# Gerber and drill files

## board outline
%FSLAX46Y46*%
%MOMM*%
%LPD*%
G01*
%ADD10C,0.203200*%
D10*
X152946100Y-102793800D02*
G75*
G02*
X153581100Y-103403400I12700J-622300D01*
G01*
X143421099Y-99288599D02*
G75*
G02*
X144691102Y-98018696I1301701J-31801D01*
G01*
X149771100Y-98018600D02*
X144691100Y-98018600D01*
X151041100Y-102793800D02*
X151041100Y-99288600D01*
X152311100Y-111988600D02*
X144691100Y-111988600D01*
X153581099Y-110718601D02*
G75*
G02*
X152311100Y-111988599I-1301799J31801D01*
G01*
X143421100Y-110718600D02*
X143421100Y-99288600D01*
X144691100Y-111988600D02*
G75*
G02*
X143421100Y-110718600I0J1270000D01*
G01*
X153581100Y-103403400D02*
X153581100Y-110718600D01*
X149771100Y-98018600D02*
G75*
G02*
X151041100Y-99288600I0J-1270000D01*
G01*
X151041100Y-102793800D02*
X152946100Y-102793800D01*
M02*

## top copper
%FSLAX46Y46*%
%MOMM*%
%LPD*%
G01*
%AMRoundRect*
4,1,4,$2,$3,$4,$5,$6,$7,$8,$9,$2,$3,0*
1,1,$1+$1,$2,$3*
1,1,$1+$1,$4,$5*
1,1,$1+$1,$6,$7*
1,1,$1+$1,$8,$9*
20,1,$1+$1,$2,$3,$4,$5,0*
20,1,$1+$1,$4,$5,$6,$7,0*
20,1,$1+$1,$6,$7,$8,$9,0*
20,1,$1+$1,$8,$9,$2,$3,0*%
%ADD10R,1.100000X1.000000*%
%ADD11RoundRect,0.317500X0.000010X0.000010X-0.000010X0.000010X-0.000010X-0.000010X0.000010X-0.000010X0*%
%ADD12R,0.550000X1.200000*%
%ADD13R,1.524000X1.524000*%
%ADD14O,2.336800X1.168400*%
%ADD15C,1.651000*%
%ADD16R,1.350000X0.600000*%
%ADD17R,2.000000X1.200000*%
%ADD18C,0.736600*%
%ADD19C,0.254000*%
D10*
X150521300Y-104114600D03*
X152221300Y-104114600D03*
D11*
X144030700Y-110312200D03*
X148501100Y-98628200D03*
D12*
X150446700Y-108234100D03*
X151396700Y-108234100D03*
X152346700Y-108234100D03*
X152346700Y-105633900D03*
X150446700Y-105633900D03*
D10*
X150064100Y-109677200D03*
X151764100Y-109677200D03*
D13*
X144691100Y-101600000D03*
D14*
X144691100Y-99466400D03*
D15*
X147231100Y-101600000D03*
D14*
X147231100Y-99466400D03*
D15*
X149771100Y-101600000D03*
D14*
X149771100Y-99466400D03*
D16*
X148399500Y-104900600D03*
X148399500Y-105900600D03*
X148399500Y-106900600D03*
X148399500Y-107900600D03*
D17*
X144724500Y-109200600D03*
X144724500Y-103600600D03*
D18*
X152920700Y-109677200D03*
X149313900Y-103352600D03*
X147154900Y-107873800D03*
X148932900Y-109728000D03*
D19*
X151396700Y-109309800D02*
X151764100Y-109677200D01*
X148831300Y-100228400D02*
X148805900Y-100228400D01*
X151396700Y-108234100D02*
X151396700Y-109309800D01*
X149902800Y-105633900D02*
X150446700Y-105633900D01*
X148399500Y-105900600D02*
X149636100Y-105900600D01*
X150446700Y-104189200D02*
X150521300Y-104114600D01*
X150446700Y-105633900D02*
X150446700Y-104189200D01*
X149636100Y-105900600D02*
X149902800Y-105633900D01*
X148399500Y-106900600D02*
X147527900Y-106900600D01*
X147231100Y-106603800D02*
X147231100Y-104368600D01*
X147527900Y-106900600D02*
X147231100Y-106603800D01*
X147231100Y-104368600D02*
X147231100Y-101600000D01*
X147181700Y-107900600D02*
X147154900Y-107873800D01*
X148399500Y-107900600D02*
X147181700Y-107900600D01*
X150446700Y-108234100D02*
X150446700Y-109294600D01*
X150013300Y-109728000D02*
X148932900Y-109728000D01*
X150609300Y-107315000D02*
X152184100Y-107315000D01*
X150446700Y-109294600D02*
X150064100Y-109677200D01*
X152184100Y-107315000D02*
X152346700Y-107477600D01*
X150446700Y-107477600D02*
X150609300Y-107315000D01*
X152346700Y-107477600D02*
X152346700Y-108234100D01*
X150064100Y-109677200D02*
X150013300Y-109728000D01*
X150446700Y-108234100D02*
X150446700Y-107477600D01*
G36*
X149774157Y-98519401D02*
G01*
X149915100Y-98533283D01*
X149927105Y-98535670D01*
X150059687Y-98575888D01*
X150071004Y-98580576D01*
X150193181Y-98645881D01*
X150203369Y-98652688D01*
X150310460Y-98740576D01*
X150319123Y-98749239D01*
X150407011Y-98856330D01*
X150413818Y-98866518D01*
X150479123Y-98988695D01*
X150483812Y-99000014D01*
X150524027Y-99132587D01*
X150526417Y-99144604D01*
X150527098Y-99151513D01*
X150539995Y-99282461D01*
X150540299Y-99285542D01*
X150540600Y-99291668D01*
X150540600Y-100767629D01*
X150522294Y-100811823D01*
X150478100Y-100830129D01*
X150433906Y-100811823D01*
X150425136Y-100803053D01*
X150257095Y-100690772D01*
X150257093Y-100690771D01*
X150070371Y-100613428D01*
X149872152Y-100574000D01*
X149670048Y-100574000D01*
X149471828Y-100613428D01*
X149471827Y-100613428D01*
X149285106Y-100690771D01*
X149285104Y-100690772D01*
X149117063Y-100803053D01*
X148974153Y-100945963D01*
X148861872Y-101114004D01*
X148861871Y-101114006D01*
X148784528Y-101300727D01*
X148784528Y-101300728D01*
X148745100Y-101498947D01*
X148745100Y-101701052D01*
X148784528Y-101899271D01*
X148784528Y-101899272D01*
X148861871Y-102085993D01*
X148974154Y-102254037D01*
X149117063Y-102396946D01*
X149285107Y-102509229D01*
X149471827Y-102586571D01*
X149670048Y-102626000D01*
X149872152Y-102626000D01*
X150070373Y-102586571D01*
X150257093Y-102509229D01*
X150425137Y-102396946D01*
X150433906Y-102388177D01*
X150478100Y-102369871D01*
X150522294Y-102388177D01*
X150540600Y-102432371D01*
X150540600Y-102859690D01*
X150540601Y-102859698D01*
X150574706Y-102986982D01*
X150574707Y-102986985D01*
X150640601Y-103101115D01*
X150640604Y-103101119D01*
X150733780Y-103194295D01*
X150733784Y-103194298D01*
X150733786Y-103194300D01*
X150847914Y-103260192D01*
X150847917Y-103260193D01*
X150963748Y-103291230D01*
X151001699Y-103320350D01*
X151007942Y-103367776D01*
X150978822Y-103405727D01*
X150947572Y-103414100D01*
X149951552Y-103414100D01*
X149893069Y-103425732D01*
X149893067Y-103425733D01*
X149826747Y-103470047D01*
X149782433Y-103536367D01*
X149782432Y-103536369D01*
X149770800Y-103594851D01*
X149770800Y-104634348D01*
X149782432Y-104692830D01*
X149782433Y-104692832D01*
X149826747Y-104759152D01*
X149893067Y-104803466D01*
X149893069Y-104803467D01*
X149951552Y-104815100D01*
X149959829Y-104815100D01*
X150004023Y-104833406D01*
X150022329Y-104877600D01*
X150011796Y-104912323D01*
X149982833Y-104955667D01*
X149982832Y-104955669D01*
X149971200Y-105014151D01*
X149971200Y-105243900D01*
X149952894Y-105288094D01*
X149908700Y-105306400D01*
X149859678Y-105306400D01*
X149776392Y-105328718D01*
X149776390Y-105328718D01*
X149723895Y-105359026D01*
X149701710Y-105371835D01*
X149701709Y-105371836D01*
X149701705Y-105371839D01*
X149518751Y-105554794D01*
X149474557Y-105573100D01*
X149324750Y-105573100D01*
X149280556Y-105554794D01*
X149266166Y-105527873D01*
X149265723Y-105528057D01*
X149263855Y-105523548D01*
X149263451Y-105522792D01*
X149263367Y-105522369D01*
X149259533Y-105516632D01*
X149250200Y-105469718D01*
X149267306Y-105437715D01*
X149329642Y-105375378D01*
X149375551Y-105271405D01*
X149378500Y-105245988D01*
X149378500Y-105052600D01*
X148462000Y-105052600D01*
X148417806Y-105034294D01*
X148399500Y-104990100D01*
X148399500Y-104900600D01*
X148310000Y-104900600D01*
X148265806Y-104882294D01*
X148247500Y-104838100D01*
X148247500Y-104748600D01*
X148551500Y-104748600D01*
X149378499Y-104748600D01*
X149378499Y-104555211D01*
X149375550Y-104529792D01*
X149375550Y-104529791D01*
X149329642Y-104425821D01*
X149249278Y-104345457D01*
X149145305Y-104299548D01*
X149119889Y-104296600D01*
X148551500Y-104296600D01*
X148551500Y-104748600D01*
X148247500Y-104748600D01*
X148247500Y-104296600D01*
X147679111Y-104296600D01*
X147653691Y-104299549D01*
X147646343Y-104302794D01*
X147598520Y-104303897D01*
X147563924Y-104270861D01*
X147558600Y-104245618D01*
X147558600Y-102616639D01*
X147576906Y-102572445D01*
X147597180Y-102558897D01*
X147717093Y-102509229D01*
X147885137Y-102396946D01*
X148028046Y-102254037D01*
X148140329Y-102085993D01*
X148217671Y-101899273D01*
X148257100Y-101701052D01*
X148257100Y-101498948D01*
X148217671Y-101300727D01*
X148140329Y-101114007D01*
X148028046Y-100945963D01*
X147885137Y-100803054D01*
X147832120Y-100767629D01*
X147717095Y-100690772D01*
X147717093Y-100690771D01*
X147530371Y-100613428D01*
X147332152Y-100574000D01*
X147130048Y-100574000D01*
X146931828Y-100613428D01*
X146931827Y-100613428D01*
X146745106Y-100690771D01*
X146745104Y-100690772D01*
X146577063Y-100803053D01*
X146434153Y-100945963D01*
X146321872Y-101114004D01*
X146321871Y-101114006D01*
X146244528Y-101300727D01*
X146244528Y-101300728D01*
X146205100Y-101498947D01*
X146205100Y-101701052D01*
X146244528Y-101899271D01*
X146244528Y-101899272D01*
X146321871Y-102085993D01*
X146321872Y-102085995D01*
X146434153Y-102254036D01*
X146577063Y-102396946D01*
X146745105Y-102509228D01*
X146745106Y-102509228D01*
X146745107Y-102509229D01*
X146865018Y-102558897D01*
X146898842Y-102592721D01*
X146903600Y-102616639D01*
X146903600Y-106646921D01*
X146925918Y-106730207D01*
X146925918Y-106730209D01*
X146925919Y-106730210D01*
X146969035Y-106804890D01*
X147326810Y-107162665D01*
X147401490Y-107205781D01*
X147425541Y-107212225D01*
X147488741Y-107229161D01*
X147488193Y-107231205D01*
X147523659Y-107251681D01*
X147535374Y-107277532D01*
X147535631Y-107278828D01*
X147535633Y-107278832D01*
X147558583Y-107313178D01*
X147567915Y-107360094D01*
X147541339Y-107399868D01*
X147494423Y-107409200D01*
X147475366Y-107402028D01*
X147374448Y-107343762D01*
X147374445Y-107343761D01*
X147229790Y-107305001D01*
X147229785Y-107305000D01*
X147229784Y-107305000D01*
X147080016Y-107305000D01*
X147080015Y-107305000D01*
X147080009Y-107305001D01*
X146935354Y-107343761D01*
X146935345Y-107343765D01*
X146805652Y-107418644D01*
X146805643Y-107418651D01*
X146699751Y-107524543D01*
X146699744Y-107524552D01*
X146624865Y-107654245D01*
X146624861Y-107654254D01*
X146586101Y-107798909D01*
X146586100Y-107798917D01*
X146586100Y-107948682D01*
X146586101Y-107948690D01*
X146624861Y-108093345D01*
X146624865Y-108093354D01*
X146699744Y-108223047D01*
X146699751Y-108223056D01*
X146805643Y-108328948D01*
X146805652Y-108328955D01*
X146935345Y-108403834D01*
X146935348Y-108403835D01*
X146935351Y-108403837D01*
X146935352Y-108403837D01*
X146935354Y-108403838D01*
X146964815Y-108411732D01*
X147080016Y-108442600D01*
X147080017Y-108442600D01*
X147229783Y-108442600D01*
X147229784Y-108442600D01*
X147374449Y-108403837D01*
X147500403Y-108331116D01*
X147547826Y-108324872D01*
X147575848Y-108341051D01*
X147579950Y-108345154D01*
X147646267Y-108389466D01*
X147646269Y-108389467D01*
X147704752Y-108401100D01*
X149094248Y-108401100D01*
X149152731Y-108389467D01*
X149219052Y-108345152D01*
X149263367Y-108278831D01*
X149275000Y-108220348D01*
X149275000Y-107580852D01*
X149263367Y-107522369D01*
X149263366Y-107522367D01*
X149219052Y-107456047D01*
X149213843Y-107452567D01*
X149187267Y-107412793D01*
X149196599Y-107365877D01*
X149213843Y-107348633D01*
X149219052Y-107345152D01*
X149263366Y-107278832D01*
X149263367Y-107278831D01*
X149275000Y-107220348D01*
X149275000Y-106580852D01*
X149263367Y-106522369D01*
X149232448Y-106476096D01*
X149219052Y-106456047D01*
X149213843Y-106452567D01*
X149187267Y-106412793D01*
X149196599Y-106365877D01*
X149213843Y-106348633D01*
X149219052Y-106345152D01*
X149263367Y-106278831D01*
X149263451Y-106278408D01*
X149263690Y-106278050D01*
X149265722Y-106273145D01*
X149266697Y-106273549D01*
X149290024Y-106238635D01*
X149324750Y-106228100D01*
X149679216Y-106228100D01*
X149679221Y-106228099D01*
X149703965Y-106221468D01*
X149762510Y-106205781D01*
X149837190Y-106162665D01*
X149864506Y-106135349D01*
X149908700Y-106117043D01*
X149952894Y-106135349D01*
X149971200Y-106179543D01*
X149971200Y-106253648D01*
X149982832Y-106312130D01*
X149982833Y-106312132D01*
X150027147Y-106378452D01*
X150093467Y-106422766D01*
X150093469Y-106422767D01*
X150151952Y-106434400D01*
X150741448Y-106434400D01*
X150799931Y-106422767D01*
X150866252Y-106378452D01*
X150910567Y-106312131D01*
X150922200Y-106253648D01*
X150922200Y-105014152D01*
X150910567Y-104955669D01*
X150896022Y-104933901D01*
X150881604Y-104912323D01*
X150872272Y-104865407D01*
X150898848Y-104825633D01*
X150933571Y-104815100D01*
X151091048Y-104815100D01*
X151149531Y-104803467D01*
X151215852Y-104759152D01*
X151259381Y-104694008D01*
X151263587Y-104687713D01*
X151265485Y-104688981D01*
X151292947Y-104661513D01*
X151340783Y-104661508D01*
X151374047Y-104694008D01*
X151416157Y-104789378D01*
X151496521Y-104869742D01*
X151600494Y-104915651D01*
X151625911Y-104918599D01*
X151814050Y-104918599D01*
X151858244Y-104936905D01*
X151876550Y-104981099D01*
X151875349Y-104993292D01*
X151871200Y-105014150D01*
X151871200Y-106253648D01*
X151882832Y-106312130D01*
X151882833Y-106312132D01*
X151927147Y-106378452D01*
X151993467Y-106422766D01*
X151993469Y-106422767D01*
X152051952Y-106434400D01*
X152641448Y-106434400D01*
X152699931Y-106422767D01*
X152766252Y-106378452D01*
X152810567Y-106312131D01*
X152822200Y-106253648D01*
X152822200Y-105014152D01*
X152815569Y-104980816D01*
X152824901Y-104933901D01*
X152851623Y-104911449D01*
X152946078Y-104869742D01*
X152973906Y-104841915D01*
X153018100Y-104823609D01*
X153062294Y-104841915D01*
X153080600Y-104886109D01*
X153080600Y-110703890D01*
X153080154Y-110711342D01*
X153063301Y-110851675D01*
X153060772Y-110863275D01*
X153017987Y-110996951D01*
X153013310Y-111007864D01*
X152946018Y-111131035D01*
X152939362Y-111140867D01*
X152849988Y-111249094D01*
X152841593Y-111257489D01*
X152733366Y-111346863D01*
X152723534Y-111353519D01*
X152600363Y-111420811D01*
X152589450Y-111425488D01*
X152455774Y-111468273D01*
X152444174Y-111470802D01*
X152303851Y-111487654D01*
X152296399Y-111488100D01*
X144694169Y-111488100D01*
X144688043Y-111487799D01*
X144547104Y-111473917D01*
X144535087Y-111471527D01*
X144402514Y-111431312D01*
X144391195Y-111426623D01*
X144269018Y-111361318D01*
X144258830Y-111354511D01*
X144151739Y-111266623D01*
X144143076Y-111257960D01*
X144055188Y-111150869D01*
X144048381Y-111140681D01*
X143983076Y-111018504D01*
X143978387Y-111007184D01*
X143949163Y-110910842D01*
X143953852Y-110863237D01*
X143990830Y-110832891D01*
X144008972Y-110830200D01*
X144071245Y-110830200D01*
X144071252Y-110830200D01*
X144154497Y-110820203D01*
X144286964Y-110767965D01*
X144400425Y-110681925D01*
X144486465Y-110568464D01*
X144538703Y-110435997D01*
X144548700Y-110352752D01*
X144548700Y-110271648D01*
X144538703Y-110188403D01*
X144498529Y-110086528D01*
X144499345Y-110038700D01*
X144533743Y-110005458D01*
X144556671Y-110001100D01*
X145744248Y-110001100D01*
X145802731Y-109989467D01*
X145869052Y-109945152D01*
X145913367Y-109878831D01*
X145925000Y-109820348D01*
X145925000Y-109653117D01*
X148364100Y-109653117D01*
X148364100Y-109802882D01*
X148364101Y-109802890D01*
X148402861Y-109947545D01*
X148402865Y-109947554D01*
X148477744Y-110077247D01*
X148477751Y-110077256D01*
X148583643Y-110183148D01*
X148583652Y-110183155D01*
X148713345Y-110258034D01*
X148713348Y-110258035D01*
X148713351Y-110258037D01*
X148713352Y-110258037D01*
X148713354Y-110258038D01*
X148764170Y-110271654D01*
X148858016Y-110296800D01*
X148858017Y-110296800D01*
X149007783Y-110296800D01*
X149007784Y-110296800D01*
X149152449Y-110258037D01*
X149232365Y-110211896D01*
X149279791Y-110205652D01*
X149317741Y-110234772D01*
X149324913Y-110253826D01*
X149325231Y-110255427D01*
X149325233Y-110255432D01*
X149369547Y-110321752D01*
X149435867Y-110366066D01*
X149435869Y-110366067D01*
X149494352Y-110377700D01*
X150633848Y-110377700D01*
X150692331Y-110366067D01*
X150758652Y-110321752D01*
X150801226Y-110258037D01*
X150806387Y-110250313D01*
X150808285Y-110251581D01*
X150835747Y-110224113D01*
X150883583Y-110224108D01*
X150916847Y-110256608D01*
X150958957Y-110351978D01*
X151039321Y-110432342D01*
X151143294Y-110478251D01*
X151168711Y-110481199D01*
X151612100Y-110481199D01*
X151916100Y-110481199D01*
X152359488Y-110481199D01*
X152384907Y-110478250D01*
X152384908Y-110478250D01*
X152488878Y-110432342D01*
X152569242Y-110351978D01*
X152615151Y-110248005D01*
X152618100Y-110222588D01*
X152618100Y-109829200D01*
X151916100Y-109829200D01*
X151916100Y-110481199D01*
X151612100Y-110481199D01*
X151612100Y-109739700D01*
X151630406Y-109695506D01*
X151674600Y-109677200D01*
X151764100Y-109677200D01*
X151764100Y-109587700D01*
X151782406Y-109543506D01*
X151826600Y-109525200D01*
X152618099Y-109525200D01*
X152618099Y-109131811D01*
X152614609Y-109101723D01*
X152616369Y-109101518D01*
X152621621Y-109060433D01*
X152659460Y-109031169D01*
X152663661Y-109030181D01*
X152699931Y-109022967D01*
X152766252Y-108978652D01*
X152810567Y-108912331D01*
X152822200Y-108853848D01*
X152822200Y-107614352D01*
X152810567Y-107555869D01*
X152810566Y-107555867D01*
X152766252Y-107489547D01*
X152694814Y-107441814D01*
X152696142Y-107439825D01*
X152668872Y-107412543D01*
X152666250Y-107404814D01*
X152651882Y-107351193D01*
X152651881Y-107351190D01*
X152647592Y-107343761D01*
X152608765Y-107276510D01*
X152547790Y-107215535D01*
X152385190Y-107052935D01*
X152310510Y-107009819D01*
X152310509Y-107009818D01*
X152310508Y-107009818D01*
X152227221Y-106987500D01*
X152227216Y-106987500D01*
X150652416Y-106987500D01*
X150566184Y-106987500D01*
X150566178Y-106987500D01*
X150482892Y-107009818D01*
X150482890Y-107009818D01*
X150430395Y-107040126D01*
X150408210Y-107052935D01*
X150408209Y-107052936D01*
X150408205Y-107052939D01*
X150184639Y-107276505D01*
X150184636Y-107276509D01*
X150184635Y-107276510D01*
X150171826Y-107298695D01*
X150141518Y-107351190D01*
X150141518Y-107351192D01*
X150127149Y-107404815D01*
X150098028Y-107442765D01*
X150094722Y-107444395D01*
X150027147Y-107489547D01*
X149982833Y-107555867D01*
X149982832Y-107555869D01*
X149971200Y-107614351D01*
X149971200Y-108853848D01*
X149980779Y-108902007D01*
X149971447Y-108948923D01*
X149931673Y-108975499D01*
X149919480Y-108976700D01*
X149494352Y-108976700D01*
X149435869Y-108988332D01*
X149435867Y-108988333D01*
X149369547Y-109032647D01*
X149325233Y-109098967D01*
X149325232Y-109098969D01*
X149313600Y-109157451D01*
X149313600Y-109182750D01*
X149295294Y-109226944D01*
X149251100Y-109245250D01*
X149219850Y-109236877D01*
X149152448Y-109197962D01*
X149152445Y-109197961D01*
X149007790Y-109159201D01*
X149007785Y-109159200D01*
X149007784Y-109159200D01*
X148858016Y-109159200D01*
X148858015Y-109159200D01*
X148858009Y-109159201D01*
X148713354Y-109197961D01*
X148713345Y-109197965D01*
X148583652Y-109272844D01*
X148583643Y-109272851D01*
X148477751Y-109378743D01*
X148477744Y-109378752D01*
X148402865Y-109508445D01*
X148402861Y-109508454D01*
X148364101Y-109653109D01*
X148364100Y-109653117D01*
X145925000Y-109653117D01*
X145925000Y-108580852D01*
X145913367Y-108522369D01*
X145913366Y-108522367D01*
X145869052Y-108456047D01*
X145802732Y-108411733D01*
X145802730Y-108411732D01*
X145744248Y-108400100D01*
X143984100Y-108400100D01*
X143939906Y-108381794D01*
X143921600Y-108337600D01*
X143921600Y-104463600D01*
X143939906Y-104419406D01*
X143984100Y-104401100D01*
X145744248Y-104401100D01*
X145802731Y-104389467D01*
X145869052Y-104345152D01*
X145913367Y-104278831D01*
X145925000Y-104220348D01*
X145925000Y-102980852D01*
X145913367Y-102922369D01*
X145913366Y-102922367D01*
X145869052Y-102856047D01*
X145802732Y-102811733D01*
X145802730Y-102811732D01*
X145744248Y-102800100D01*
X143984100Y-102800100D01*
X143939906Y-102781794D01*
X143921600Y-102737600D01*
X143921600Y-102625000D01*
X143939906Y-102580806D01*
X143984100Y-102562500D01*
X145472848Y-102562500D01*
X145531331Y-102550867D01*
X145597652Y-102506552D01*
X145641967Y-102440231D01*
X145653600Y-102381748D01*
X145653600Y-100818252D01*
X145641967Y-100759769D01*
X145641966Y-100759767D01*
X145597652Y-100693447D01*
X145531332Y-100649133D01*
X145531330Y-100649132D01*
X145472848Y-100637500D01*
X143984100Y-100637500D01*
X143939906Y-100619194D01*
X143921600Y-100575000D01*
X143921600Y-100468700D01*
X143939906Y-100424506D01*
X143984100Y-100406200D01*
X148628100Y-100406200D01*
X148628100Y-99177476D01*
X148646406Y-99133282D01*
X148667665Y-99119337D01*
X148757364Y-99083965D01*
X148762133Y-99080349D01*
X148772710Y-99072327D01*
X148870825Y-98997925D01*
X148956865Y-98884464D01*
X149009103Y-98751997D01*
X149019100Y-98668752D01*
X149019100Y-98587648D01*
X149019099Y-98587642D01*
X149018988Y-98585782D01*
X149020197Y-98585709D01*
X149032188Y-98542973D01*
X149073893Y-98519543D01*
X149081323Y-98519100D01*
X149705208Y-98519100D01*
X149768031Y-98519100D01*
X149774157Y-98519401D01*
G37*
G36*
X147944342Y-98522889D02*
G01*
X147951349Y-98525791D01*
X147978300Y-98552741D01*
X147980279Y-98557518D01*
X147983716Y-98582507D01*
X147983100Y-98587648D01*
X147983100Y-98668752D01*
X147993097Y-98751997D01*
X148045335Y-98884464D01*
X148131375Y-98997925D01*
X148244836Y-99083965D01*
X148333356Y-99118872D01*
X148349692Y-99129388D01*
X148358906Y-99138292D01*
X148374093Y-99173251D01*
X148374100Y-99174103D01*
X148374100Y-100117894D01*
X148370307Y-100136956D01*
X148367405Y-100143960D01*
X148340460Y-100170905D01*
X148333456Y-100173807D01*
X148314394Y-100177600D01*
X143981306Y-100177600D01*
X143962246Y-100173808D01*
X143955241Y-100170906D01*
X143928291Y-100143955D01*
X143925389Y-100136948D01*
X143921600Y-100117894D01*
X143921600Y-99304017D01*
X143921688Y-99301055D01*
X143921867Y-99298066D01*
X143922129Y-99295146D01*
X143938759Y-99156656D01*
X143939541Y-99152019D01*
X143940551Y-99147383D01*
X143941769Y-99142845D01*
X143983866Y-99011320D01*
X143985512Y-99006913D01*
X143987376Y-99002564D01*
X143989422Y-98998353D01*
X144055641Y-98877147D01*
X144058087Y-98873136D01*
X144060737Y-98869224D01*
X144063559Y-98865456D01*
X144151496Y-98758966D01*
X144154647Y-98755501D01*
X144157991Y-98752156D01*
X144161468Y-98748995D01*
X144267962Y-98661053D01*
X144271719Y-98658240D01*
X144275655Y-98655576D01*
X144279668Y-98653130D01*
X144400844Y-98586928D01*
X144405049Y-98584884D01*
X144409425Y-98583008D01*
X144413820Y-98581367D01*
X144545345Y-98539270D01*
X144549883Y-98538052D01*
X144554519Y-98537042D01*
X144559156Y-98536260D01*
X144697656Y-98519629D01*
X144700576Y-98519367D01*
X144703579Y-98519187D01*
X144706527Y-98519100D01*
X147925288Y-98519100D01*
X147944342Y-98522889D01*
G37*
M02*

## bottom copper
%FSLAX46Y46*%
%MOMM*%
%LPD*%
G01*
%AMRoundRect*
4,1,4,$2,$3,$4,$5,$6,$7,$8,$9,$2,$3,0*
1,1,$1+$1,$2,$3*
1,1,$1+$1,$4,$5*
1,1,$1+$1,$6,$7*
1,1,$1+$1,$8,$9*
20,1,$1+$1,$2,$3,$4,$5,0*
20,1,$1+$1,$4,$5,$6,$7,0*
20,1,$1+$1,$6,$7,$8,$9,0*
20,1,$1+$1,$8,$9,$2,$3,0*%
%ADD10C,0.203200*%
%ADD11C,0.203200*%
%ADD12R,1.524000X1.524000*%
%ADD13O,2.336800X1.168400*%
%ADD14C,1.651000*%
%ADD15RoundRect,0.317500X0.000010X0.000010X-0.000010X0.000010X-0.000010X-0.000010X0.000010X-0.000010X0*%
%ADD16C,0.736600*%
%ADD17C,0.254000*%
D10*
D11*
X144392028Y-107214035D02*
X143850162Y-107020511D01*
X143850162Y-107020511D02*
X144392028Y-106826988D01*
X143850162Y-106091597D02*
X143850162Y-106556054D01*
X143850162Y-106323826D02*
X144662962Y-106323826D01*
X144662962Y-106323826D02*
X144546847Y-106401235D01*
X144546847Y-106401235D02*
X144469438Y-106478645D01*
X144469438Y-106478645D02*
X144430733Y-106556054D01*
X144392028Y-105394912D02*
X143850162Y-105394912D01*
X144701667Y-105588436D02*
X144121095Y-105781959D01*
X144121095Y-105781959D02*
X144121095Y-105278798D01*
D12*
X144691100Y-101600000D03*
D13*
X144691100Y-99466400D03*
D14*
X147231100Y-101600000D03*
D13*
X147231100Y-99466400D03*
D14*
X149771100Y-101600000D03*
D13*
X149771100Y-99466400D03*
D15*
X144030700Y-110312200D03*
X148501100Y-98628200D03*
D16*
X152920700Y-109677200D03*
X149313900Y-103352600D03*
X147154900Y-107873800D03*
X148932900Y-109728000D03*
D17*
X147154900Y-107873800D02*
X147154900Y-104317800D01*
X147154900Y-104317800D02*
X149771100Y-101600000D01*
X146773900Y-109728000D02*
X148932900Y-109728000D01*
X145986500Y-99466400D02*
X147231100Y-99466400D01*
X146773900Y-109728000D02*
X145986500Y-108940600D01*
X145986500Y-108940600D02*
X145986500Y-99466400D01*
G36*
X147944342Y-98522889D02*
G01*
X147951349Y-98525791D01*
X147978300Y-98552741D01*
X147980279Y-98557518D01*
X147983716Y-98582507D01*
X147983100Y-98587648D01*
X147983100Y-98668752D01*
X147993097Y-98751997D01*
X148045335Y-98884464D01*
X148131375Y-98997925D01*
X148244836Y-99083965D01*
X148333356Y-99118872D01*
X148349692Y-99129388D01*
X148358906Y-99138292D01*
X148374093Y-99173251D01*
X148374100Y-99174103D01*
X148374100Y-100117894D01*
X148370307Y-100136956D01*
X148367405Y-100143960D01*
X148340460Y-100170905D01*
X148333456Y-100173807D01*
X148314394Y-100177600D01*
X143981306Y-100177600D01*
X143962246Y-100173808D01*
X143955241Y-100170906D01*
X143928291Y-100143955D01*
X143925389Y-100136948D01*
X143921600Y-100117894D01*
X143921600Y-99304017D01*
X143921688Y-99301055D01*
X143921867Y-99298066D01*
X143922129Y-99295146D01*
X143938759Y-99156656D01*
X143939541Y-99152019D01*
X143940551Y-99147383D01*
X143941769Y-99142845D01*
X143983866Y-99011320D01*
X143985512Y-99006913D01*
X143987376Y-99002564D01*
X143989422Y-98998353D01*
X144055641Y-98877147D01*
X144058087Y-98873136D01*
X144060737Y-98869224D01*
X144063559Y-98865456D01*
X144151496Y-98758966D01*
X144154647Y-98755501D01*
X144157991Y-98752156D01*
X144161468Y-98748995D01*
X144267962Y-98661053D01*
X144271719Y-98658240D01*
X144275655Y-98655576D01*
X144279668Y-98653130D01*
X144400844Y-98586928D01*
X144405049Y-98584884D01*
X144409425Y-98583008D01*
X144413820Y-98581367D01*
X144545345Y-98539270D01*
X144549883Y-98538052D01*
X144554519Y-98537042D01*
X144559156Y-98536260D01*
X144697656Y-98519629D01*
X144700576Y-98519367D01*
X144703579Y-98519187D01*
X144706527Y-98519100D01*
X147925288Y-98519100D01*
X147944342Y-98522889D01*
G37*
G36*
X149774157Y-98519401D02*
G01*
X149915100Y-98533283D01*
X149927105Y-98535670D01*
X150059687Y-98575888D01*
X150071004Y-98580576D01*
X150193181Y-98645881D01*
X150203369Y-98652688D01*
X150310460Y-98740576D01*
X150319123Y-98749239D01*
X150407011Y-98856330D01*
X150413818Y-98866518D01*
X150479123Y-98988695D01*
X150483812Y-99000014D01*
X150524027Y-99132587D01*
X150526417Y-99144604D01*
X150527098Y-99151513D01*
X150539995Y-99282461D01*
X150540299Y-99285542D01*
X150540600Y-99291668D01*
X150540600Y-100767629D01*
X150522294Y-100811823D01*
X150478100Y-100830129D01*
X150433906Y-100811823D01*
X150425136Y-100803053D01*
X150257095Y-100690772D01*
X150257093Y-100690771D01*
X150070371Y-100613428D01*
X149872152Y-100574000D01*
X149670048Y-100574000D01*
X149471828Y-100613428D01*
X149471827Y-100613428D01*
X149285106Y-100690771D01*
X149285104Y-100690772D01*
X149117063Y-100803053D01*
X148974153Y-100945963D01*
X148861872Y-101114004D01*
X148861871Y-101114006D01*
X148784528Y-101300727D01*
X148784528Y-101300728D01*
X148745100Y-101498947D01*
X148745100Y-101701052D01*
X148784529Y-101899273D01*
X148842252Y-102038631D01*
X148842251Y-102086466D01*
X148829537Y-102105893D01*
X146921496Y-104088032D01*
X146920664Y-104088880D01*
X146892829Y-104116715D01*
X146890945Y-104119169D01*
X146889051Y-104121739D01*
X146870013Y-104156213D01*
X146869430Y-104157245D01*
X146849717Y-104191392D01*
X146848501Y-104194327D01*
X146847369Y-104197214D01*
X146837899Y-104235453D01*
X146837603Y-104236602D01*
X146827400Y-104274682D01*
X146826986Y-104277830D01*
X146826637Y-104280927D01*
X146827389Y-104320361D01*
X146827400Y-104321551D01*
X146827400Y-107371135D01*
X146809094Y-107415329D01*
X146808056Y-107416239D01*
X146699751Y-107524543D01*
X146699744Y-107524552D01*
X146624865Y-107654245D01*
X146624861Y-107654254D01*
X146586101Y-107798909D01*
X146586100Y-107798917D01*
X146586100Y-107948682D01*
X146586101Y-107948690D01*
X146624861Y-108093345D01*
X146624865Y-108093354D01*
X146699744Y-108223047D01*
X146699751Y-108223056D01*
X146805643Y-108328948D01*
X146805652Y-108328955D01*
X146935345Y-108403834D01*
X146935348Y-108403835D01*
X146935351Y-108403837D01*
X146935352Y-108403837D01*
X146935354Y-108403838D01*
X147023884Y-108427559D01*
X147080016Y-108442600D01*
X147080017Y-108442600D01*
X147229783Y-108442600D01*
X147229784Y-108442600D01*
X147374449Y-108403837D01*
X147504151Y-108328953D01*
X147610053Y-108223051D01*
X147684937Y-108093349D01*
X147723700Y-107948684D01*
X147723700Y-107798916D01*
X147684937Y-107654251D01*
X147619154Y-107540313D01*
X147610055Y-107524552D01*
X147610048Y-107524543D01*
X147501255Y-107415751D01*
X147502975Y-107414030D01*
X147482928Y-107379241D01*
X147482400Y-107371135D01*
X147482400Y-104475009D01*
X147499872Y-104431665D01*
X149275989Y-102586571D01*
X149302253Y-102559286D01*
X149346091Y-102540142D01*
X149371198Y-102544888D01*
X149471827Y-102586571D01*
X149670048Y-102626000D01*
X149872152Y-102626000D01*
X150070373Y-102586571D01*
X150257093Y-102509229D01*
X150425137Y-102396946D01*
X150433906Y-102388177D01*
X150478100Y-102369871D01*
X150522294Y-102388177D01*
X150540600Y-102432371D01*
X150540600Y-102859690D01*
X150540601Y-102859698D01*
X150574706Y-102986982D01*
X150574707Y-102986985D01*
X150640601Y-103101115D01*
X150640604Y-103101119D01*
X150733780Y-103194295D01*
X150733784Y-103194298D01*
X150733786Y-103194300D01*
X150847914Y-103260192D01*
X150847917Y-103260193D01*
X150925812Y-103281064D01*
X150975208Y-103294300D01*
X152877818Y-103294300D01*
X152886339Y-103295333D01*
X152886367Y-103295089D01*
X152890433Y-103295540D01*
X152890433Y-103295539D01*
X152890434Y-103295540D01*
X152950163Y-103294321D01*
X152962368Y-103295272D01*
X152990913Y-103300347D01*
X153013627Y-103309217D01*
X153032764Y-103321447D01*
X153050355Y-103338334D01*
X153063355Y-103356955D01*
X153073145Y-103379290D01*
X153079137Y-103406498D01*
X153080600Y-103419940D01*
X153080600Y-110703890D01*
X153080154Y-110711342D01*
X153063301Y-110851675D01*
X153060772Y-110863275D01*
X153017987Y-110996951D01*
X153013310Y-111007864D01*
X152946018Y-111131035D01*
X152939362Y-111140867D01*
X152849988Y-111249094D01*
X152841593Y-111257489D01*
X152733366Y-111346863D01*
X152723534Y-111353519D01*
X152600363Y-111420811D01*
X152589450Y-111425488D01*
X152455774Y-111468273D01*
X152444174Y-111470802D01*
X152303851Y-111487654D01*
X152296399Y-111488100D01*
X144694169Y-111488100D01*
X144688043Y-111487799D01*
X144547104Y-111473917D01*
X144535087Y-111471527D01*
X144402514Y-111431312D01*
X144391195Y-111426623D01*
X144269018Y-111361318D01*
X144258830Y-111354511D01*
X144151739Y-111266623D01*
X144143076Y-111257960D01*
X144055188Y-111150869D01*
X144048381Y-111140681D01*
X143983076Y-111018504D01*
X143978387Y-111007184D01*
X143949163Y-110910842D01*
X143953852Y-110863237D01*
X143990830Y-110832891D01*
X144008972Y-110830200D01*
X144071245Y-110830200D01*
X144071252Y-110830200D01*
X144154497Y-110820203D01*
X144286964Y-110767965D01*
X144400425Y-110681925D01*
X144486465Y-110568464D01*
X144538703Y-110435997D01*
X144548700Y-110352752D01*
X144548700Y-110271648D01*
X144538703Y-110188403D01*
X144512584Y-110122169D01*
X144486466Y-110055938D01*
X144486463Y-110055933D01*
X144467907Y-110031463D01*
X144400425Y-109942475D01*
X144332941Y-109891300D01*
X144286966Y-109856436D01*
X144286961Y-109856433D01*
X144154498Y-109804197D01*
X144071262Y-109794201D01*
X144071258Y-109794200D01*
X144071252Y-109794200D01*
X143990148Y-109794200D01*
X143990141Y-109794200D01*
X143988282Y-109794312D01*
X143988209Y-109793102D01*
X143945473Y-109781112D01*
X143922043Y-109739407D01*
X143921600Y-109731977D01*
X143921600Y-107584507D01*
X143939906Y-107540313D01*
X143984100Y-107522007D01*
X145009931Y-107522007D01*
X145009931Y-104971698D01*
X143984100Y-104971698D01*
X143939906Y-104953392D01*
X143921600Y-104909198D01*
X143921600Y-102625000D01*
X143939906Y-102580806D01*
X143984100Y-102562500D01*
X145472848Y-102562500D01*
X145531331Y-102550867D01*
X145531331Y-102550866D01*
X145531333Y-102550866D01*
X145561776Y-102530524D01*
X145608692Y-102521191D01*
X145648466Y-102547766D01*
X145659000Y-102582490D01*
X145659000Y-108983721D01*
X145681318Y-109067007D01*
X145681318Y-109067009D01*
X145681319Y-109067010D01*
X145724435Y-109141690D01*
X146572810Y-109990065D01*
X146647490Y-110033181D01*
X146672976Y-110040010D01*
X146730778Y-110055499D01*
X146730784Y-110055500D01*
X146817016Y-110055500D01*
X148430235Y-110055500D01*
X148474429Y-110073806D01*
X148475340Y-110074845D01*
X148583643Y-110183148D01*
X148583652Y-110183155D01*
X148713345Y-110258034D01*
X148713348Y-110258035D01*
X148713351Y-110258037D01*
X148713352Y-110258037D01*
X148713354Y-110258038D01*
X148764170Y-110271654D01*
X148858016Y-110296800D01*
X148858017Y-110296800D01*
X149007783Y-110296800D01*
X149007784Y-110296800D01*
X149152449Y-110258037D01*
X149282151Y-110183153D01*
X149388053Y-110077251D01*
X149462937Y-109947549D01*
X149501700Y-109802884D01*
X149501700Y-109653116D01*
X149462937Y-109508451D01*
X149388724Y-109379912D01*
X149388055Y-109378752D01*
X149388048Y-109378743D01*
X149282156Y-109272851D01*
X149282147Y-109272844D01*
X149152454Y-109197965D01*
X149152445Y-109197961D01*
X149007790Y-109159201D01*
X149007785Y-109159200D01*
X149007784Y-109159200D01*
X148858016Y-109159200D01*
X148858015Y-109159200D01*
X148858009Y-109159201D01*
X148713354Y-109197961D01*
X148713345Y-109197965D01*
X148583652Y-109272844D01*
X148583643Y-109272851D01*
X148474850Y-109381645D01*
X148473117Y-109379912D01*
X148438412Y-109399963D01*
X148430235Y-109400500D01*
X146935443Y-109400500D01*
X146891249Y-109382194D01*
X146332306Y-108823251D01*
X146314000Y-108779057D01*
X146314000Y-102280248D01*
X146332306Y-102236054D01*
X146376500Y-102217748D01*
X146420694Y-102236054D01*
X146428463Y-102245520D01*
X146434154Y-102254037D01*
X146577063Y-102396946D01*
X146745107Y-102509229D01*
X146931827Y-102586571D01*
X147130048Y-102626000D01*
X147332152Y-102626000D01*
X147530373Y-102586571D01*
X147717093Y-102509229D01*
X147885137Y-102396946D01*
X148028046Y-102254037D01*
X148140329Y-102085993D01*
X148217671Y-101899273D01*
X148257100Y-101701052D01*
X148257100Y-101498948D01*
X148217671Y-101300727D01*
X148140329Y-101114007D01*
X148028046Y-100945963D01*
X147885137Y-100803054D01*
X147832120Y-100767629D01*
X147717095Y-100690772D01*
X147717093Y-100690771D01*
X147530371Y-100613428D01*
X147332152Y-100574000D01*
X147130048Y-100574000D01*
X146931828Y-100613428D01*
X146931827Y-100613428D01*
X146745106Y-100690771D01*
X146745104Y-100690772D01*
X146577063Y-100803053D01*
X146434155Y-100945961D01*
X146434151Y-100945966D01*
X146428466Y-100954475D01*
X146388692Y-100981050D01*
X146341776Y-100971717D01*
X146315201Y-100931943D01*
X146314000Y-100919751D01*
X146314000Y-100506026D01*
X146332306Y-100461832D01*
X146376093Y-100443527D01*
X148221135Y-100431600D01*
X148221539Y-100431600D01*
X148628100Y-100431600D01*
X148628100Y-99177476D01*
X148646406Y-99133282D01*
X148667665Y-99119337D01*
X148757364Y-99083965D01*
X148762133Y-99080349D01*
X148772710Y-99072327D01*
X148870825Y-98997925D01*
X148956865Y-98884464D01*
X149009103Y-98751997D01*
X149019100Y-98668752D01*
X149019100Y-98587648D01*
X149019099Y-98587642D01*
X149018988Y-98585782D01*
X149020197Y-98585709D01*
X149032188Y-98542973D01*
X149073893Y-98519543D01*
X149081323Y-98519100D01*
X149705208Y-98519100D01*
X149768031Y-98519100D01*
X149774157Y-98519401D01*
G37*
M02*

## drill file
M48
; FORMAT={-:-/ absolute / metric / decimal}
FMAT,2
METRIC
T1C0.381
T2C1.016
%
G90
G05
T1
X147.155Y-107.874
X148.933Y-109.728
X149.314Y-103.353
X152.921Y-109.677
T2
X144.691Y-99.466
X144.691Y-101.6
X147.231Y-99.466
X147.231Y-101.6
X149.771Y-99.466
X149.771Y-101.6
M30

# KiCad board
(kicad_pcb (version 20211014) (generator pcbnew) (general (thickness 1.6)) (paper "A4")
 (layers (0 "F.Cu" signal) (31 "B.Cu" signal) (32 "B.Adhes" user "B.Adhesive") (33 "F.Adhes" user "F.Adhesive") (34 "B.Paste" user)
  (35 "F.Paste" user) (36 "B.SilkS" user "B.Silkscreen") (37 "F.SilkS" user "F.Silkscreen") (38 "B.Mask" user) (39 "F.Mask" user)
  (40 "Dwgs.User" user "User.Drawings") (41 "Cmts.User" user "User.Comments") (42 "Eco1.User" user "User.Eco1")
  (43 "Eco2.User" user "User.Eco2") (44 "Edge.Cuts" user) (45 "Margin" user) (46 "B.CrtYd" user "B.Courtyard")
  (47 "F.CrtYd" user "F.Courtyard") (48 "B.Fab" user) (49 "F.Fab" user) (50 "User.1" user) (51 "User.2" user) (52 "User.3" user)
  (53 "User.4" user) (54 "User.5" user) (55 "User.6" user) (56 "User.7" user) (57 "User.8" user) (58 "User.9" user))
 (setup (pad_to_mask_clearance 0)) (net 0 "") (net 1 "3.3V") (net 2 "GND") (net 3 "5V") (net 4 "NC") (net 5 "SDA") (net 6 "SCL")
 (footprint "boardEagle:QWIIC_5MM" (layer "F.Cu") (at 146.8501 110.8456)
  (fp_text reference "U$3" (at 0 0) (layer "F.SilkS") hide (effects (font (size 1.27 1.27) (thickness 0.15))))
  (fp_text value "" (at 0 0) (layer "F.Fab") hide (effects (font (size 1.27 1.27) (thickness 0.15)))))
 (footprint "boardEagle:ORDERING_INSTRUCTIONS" (layer "F.Cu") (at 111.6711 127.2286)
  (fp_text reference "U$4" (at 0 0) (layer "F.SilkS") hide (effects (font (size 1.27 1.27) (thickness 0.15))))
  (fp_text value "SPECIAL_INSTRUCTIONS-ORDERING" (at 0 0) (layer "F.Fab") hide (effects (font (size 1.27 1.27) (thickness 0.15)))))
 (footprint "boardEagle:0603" (layer "F.Cu") (at 151.3713 104.1146)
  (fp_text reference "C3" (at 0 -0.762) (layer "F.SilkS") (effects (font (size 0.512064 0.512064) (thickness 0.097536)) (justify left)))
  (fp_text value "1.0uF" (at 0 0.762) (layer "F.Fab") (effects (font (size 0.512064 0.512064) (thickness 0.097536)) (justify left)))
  (pad "1" smd rect (at -0.85 0) (size 1.1 1) (layers "F.Cu" "F.Paste" "F.Mask") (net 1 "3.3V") (solder_mask_margin 0.1016))
  (pad "2" smd rect (at 0.85 0) (size 1.1 1) (layers "F.Cu" "F.Paste" "F.Mask") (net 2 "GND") (solder_mask_margin 0.1016)))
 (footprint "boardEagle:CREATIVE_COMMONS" (layer "F.Cu") (at 131.9911 125.9586)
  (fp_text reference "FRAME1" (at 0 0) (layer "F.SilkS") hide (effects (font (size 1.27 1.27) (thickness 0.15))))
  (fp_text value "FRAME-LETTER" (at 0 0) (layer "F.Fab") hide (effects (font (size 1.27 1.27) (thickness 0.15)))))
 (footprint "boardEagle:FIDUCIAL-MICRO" (layer "F.Cu") (at 144.0307 110.3122 180)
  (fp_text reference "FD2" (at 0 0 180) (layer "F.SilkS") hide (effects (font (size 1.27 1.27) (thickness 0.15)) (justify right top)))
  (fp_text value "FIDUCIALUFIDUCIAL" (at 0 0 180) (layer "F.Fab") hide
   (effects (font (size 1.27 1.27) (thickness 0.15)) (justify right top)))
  (pad "1" smd roundrect (at 0 0 180) (size 0.635 0.635) (layers "F.Cu" "F.Mask") (roundrect_rratio 0.5) (solder_mask_margin 0.1016)))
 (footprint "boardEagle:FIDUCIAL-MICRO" (layer "F.Cu") (at 148.5011 98.6282 180)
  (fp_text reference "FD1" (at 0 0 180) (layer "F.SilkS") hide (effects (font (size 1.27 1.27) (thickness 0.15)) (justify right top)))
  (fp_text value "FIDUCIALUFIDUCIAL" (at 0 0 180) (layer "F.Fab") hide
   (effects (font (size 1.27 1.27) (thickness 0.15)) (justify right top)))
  (pad "1" smd roundrect (at 0 0 180) (size 0.635 0.635) (layers "F.Cu" "F.Mask") (roundrect_rratio 0.5) (solder_mask_margin 0.1016)))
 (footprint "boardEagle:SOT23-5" (layer "F.Cu") (at 151.3967 106.934)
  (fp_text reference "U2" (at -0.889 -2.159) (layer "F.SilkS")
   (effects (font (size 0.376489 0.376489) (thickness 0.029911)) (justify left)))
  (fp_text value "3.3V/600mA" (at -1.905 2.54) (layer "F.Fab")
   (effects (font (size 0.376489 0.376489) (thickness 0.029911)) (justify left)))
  (pad "1" smd rect (at -0.95 1.3001) (size 0.55 1.2) (layers "F.Cu" "F.Paste" "F.Mask") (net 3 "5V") (solder_mask_margin 0.1016))
  (pad "2" smd rect (at 0 1.3001) (size 0.55 1.2) (layers "F.Cu" "F.Paste" "F.Mask") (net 2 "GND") (solder_mask_margin 0.1016))
  (pad "3" smd rect (at 0.95 1.3001) (size 0.55 1.2) (layers "F.Cu" "F.Paste" "F.Mask") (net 3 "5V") (solder_mask_margin 0.1016))
  (pad "4" smd rect (at 0.95 -1.3001) (size 0.55 1.2) (layers "F.Cu" "F.Paste" "F.Mask") (solder_mask_margin 0.1016))
  (pad "5" smd rect (at -0.95 -1.3001) (size 0.55 1.2) (layers "F.Cu" "F.Paste" "F.Mask") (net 1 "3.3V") (solder_mask_margin 0.1016)))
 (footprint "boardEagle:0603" (layer "F.Cu") (at 150.9141 109.6772)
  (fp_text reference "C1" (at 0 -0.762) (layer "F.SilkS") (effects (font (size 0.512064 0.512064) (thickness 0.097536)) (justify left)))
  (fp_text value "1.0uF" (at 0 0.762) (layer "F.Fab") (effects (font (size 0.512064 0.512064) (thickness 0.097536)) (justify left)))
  (pad "1" smd rect (at -0.85 0) (size 1.1 1) (layers "F.Cu" "F.Paste" "F.Mask") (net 3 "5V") (solder_mask_margin 0.1016))
  (pad "2" smd rect (at 0.85 0) (size 1.1 1) (layers "F.Cu" "F.Paste" "F.Mask") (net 2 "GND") (solder_mask_margin 0.1016)))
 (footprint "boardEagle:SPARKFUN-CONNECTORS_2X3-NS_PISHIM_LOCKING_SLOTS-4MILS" (layer "F.Cu") (at 147.2311 100.5586)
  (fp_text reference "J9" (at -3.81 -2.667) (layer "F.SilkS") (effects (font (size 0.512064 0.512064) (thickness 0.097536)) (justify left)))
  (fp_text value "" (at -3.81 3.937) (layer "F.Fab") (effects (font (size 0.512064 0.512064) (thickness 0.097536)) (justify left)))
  (pad "1" thru_hole rect (at -2.54 1.0414) (size 1.524 1.524) (drill 1.016) (layers *.Cu *.Mask) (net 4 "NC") (solder_mask_margin 0.1016))
  (pad "2" thru_hole oval (at -2.54 -1.0922) (size 2.3368 1.1684) (drill 1.016) (layers *.Cu) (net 3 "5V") (solder_mask_margin 0.1016)
   (zone_connect 2))
  (pad "3" thru_hole circle (at 0 1.0414) (size 1.651 1.651) (drill 1.016) (layers *.Cu *.Mask) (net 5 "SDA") (solder_mask_margin 0.1016))
  (pad "4" thru_hole oval (at 0 -1.0922) (size 2.3368 1.1684) (drill 1.016) (layers *.Cu) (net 3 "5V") (solder_mask_margin 0.1016)
   (zone_connect 2))
  (pad "5" thru_hole circle (at 2.54 1.0414) (size 1.651 1.651) (drill 1.016) (layers *.Cu *.Mask) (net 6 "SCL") (solder_mask_margin 0.1016))
  (pad "6" thru_hole oval (at 2.54 -1.0922) (size 2.3368 1.1684) (drill 1.016) (layers *.Cu) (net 2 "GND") (solder_mask_margin 0.1016)
   (zone_connect 2)))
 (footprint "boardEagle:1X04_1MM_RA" (layer "F.Cu") (at 148.3995 106.4006 -90)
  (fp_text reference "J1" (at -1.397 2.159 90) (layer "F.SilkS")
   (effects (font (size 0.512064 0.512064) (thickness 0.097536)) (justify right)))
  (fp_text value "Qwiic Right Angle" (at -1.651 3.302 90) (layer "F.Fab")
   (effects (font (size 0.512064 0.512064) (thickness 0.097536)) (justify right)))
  (pad "1" smd rect (at -1.5 0 270) (size 0.6 1.35) (layers "F.Cu" "F.Paste" "F.Mask") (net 2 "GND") (solder_mask_margin 0.1016))
  (pad "2" smd rect (at -0.5 0 270) (size 0.6 1.35) (layers "F.Cu" "F.Paste" "F.Mask") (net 1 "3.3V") (solder_mask_margin 0.1016))
  (pad "3" smd rect (at 0.5 0 270) (size 0.6 1.35) (layers "F.Cu" "F.Paste" "F.Mask") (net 5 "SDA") (solder_mask_margin 0.1016))
  (pad "4" smd rect (at 1.5 0 270) (size 0.6 1.35) (layers "F.Cu" "F.Paste" "F.Mask") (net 6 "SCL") (solder_mask_margin 0.1016))
  (pad "NC1" smd rect (at 2.8 3.675 270) (size 1.2 2) (layers "F.Cu" "F.Paste" "F.Mask") (solder_mask_margin 0.1016))
  (pad "NC2" smd rect (at -2.8 3.675 270) (size 1.2 2) (layers "F.Cu" "F.Paste" "F.Mask") (solder_mask_margin 0.1016)))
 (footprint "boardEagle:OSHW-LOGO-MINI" (layer "B.Cu") (at 146.0119 110.363 180)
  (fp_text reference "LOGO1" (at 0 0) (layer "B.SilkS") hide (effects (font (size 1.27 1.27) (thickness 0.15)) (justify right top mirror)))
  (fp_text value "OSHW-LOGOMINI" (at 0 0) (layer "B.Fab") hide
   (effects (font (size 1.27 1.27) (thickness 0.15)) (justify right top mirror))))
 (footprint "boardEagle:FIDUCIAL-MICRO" (layer "B.Cu") (at 144.0307 110.3122 180)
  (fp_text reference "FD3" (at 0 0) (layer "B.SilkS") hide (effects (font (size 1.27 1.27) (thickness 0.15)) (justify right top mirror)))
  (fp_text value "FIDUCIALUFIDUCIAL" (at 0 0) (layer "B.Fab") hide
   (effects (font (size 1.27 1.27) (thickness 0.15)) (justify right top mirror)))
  (pad "1" smd roundrect (at 0 0 180) (size 0.635 0.635) (layers "B.Cu" "B.Mask") (roundrect_rratio 0.5) (solder_mask_margin 0.1016)))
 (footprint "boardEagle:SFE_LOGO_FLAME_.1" (layer "B.Cu") (at 152.8445 111.633 180)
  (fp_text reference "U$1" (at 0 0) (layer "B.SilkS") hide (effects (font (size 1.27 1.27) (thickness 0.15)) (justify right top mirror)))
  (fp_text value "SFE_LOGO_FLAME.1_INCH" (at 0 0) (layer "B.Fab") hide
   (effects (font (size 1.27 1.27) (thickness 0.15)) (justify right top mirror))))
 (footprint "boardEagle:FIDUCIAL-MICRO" (layer "B.Cu") (at 148.5011 98.6282 180)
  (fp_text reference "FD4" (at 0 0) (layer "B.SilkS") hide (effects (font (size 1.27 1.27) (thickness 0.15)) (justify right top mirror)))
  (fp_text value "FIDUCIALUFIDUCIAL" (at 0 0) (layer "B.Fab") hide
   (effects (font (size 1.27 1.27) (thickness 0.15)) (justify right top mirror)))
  (pad "1" smd roundrect (at 0 0 180) (size 0.635 0.635) (layers "B.Cu" "B.Mask") (roundrect_rratio 0.5) (solder_mask_margin 0.1016)))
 (gr_arc (start 152.9461 102.7938) (mid 153.389852 102.967087) (end 153.5811 103.4034) (layer "Edge.Cuts") (width 0.2032))
 (gr_arc (start 143.421099 99.288599) (mid 143.8021 98.399599) (end 144.6911 98.0186) (layer "Edge.Cuts") (width 0.2032))
 (gr_line (start 149.7711 98.0186) (end 144.6911 98.0186) (layer "Edge.Cuts") (width 0.2032))
 (gr_line (start 151.0411 102.7938) (end 151.0411 99.2886) (layer "Edge.Cuts") (width 0.2032))
 (gr_line (start 152.3111 111.9886) (end 144.6911 111.9886) (layer "Edge.Cuts") (width 0.2032))
 (gr_arc (start 153.581099 110.718601) (mid 153.200099 111.6076) (end 152.3111 111.9886) (layer "Edge.Cuts") (width 0.2032))
 (gr_line (start 143.4211 110.7186) (end 143.4211 99.2886) (layer "Edge.Cuts") (width 0.2032))
 (gr_arc (start 144.6911 111.9886) (mid 143.793074 111.616626) (end 143.4211 110.7186) (layer "Edge.Cuts") (width 0.2032))
 (gr_line (start 153.5811 103.4034) (end 153.5811 110.7186) (layer "Edge.Cuts") (width 0.2032))
 (gr_arc (start 149.7711 98.0186) (mid 150.669126 98.390574) (end 151.0411 99.2886) (layer "Edge.Cuts") (width 0.2032))
 (gr_line (start 151.0411 102.7938) (end 152.9461 102.7938) (layer "Edge.Cuts") (width 0.2032))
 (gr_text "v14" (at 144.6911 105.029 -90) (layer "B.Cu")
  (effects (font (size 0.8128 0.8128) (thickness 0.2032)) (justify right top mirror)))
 (segment (start 151.3967 109.3098) (end 151.7641 109.6772) (width 0.254) (layer "F.Cu") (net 2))
 (segment (start 148.8313 100.2284) (end 148.8059 100.2284) (width 0.254) (layer "F.Cu") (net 2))
 (segment (start 151.3967 108.2341) (end 151.3967 109.3098) (width 0.254) (layer "F.Cu") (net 2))
 (via (at 152.9207 109.6772) (size 0.7366) (drill 0.381) (layers "F.Cu" "B.Cu") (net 2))
 (via (at 149.3139 103.3526) (size 0.7366) (drill 0.381) (layers "F.Cu" "B.Cu") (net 2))
 (segment (start 149.9028 105.6339) (end 150.4467 105.6339) (width 0.254) (layer "F.Cu") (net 1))
 (segment (start 148.3995 105.9006) (end 149.6361 105.9006) (width 0.254) (layer "F.Cu") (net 1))
 (segment (start 150.4467 104.1892) (end 150.5213 104.1146) (width 0.254) (layer "F.Cu") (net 1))
 (segment (start 150.4467 105.6339) (end 150.4467 104.1892) (width 0.254) (layer "F.Cu") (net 1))
 (segment (start 149.6361 105.9006) (end 149.9028 105.6339) (width 0.254) (layer "F.Cu") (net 1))
 (segment (start 148.3995 106.9006) (end 147.5279 106.9006) (width 0.254) (layer "F.Cu") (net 5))
 (segment (start 147.2311 106.6038) (end 147.2311 104.3686) (width 0.254) (layer "F.Cu") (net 5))
 (segment (start 147.5279 106.9006) (end 147.2311 106.6038) (width 0.254) (layer "F.Cu") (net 5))
 (segment (start 147.2311 104.3686) (end 147.2311 101.6) (width 0.254) (layer "F.Cu") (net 5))
 (segment (start 147.1817 107.9006) (end 147.1549 107.8738) (width 0.254) (layer "F.Cu") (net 6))
 (segment (start 148.3995 107.9006) (end 147.1817 107.9006) (width 0.254) (layer "F.Cu") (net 6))
 (via (at 147.1549 107.8738) (size 0.7366) (drill 0.381) (layers "F.Cu" "B.Cu") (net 6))
 (segment (start 147.1549 107.8738) (end 147.1549 104.3178) (width 0.254) (layer "B.Cu") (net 6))
 (segment (start 147.1549 104.3178) (end 149.7711 101.6) (width 0.254) (layer "B.Cu") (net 6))
 (segment (start 150.4467 108.2341) (end 150.4467 109.2946) (width 0.254) (layer "F.Cu") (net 3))
 (segment (start 150.0133 109.728) (end 148.9329 109.728) (width 0.254) (layer "F.Cu") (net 3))
 (segment (start 150.6093 107.315) (end 152.1841 107.315) (width 0.254) (layer "F.Cu") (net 3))
 (segment (start 150.4467 109.2946) (end 150.0641 109.6772) (width 0.254) (layer "F.Cu") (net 3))
 (segment (start 152.1841 107.315) (end 152.3467 107.4776) (width 0.254) (layer "F.Cu") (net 3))
 (segment (start 150.4467 107.4776) (end 150.6093 107.315) (width 0.254) (layer "F.Cu") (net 3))
 (segment (start 152.3467 107.4776) (end 152.3467 108.2341) (width 0.254) (layer "F.Cu") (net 3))
 (segment (start 150.0641 109.6772) (end 150.0133 109.728) (width 0.254) (layer "F.Cu") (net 3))
 (segment (start 150.4467 108.2341) (end 150.4467 107.4776) (width 0.254) (layer "F.Cu") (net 3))
 (via (at 148.9329 109.728) (size 0.7366) (drill 0.381) (layers "F.Cu" "B.Cu") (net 3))
 (segment (start 146.7739 109.728) (end 148.9329 109.728) (width 0.254) (layer "B.Cu") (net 3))
 (segment (start 145.9865 99.4664) (end 147.2311 99.4664) (width 0.254) (layer "B.Cu") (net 3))
 (segment (start 146.7739 109.728) (end 145.9865 108.9406) (width 0.254) (layer "B.Cu") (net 3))
 (segment (start 145.9865 108.9406) (end 145.9865 99.4664) (width 0.254) (layer "B.Cu") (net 3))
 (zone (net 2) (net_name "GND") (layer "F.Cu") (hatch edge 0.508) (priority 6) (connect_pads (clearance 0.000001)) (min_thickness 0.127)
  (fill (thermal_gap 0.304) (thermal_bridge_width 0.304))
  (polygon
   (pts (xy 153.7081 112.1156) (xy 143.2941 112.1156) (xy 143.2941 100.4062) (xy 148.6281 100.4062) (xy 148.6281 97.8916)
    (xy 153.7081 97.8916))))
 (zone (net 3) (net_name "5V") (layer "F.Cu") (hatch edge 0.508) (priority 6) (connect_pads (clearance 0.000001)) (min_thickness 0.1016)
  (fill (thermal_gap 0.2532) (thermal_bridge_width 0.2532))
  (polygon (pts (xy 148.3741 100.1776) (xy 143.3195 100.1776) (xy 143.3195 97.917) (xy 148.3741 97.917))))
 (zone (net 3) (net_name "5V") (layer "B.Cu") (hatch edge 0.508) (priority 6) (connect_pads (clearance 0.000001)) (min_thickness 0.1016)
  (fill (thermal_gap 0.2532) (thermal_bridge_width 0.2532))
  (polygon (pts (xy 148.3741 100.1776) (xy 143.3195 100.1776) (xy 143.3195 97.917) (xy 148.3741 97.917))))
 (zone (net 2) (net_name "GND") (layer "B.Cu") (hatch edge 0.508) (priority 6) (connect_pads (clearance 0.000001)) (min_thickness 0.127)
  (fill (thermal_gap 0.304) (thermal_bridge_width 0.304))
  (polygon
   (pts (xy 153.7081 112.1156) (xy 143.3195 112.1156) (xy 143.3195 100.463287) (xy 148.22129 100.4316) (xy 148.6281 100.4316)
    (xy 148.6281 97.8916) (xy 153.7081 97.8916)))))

